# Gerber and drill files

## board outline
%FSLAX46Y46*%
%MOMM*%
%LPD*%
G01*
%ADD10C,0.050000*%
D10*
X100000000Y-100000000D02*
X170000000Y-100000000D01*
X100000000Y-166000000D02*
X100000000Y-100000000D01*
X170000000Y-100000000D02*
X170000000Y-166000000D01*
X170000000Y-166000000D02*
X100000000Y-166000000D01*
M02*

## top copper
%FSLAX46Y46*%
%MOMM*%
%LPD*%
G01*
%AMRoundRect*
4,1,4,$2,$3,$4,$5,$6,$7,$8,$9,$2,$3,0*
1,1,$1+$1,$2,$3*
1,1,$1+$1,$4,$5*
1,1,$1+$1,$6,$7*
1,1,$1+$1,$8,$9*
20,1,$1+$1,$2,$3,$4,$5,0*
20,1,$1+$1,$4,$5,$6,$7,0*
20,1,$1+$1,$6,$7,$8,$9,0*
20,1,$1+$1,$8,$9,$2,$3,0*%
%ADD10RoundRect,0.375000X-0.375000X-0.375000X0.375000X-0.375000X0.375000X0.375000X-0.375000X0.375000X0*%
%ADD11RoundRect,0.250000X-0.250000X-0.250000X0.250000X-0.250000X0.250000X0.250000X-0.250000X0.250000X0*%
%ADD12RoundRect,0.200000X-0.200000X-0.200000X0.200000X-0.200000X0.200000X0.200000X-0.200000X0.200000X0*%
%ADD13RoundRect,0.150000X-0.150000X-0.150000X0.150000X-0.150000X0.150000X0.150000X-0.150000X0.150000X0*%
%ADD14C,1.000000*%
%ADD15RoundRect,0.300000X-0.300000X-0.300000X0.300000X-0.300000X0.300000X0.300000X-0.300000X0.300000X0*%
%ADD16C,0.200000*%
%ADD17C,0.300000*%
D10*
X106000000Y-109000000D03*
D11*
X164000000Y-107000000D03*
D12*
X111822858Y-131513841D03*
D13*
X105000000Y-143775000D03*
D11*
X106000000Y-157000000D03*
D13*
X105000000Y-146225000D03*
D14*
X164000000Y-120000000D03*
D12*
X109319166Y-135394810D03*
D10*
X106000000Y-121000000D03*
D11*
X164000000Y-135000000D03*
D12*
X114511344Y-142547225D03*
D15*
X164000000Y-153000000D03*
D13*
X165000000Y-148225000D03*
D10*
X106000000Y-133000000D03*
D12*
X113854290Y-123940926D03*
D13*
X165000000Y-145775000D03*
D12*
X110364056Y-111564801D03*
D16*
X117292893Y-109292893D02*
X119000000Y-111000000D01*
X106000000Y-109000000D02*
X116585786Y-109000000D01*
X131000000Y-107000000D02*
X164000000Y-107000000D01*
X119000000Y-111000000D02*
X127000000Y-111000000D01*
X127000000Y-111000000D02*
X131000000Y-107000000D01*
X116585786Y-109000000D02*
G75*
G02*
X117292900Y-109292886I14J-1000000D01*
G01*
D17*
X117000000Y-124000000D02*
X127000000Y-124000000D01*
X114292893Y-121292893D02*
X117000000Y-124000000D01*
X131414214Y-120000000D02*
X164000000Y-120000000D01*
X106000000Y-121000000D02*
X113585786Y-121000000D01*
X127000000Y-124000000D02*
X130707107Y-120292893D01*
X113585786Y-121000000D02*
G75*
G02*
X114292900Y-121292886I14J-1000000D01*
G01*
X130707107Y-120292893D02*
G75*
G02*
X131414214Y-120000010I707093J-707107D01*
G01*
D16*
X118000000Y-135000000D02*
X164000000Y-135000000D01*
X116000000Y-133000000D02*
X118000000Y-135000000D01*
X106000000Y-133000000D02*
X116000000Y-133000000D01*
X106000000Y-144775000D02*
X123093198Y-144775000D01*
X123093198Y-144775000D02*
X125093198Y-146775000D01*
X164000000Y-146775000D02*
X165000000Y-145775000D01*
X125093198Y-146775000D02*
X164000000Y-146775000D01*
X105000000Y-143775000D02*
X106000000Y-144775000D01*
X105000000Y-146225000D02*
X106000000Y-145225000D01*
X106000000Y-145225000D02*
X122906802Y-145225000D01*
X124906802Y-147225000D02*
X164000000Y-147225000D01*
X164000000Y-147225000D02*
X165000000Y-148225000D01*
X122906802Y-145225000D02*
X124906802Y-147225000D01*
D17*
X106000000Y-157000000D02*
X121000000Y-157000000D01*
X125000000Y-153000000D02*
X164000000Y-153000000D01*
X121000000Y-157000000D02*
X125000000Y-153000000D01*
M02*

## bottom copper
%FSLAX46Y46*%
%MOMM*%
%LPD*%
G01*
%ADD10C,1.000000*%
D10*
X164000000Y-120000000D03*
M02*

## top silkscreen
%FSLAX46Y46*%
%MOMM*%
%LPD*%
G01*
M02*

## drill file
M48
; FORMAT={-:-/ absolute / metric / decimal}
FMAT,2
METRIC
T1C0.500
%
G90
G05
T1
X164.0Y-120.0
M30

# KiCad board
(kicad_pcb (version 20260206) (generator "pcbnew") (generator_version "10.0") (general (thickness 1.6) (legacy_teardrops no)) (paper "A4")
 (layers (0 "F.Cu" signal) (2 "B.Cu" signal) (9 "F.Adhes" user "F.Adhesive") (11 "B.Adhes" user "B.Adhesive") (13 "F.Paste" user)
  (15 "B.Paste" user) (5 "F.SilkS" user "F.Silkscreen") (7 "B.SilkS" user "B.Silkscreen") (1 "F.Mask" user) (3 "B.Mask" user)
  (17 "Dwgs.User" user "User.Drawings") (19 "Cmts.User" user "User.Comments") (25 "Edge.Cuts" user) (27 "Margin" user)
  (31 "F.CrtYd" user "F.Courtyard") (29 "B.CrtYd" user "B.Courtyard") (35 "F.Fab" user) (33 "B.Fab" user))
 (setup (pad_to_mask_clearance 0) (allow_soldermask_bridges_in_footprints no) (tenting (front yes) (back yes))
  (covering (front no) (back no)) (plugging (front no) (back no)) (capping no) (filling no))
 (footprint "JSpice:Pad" (layer "F.Cu") (at 106 109)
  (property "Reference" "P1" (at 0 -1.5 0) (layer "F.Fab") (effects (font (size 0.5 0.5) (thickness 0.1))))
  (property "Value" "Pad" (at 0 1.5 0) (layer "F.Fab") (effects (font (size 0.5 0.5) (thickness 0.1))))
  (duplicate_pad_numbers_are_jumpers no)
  (pad "1" smd roundrect (at 0 0) (size 1.5 1.5) (layers "F.Cu" "F.Mask") (roundrect_rratio 0.25) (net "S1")))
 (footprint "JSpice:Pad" (layer "F.Cu") (at 164 107)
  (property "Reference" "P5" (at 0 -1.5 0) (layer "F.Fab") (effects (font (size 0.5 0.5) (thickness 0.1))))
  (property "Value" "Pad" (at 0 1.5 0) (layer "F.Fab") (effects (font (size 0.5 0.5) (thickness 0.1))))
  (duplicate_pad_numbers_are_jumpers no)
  (pad "1" smd roundrect (at 0 0) (size 1 1) (layers "F.Cu" "F.Mask") (roundrect_rratio 0.25) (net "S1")))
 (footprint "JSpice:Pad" (layer "F.Cu") (at 111.822858 131.513841)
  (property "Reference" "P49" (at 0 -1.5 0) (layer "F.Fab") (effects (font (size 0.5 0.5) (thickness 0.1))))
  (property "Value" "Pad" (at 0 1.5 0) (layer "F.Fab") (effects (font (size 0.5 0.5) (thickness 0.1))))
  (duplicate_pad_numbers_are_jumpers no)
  (pad "1" smd roundrect (at 0 0) (size 0.8 0.8) (layers "F.Cu" "F.Mask") (roundrect_rratio 0.25) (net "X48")))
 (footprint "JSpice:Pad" (layer "F.Cu") (at 105 143.775)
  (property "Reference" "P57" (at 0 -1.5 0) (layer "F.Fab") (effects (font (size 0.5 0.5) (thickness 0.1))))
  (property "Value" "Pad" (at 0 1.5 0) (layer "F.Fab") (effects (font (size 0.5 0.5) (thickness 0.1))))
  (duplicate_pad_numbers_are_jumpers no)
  (pad "1" smd roundrect (at 0 0) (size 0.6 0.6) (layers "F.Cu" "F.Mask") (roundrect_rratio 0.25) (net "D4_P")))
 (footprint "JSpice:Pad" (layer "F.Cu") (at 106 157)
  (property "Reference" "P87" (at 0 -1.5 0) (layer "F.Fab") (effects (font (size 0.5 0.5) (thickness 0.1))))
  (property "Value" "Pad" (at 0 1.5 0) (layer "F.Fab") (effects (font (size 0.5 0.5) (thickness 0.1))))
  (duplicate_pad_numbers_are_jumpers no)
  (pad "1" smd roundrect (at 0 0) (size 1 1) (layers "F.Cu" "F.Mask") (roundrect_rratio 0.25) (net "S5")))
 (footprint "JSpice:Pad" (layer "F.Cu") (at 105 146.225)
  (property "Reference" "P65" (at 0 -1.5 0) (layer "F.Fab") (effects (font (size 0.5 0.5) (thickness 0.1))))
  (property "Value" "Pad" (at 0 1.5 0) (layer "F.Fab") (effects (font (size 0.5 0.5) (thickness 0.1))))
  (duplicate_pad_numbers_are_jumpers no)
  (pad "1" smd roundrect (at 0 0) (size 0.6 0.6) (layers "F.Cu" "F.Mask") (roundrect_rratio 0.25) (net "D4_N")))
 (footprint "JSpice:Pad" (layer "F.Cu") (at 164 120)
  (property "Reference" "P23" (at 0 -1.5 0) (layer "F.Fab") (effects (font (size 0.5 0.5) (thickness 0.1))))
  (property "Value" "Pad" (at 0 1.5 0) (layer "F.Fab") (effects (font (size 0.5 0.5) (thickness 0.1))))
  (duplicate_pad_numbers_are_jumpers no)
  (pad "1" thru_hole circle (at 0 0) (size 1 1) (drill 0.5) (layers "*.Cu" "*.Mask") (remove_unused_layers no) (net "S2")))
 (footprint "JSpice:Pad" (layer "F.Cu") (at 109.319166 135.39481)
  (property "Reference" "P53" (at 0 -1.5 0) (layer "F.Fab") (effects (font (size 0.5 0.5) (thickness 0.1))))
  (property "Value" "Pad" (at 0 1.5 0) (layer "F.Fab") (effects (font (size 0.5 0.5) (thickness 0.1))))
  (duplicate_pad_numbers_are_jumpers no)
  (pad "1" smd roundrect (at 0 0) (size 0.8 0.8) (layers "F.Cu" "F.Mask") (roundrect_rratio 0.25) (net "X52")))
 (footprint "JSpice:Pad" (layer "F.Cu") (at 106 121)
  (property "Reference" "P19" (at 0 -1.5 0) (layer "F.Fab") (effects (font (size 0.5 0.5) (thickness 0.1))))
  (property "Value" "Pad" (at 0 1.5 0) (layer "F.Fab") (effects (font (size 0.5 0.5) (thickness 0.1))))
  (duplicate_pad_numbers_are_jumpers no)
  (pad "1" smd roundrect (at 0 0) (size 1.5 1.5) (layers "F.Cu" "F.Mask") (roundrect_rratio 0.25) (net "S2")))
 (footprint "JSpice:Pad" (layer "F.Cu") (at 164 135)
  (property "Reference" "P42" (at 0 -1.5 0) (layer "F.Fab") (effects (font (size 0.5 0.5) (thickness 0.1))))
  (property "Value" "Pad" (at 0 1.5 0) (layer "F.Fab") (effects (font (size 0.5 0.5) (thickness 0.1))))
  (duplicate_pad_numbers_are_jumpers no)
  (pad "1" smd roundrect (at 0 0) (size 1 1) (layers "F.Cu" "F.Mask") (roundrect_rratio 0.25) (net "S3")))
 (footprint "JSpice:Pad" (layer "F.Cu") (at 114.511344 142.547225)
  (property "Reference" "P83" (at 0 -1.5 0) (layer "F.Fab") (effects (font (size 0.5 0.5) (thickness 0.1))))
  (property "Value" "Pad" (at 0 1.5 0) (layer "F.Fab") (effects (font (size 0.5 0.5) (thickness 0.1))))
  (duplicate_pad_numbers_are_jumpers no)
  (pad "1" smd roundrect (at 0 0) (size 0.8 0.8) (layers "F.Cu" "F.Mask") (roundrect_rratio 0.25) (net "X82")))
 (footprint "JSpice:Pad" (layer "F.Cu") (at 164 153)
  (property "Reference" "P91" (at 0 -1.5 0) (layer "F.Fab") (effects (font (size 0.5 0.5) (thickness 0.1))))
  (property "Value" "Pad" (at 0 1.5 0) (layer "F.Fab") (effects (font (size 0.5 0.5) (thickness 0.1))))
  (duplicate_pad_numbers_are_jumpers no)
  (pad "1" smd roundrect (at 0 0) (size 1.2 1.2) (layers "F.Cu" "F.Mask") (roundrect_rratio 0.25) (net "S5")))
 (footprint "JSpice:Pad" (layer "F.Cu") (at 165 148.225)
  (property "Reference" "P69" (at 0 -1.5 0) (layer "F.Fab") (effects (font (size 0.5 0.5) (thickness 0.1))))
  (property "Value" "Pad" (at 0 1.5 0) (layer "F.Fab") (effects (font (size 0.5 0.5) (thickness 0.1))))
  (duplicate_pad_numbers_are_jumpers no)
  (pad "1" smd roundrect (at 0 0) (size 0.6 0.6) (layers "F.Cu" "F.Mask") (roundrect_rratio 0.25) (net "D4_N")))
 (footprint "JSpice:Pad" (layer "F.Cu") (at 106 133)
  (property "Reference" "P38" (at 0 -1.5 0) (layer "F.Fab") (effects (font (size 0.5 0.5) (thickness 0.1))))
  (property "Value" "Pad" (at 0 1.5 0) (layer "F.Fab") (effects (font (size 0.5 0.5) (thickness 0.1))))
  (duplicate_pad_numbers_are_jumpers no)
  (pad "1" smd roundrect (at 0 0) (size 1.5 1.5) (layers "F.Cu" "F.Mask") (roundrect_rratio 0.25) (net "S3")))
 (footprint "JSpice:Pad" (layer "F.Cu") (at 113.85429 123.940926)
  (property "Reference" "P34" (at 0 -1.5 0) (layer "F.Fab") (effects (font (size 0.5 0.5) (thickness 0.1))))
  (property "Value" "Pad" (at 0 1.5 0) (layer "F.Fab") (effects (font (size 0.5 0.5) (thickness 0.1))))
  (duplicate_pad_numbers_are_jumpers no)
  (pad "1" smd roundrect (at 0 0) (size 0.8 0.8) (layers "F.Cu" "F.Mask") (roundrect_rratio 0.25) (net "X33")))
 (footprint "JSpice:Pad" (layer "F.Cu") (at 165 145.775)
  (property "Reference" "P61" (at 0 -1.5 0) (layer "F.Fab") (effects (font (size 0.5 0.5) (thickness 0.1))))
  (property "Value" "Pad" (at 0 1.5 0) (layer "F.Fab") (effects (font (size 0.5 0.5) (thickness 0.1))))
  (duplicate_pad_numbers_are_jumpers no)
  (pad "1" smd roundrect (at 0 0) (size 0.6 0.6) (layers "F.Cu" "F.Mask") (roundrect_rratio 0.25) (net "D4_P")))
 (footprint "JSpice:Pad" (layer "F.Cu") (at 110.364056 111.564801)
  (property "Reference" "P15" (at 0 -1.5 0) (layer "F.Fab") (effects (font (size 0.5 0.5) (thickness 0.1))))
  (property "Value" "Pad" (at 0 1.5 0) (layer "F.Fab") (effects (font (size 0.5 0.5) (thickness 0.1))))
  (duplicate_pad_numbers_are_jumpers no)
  (pad "1" smd roundrect (at 0 0) (size 0.8 0.8) (layers "F.Cu" "F.Mask") (roundrect_rratio 0.25) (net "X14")))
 (gr_line (start 100 100) (end 170 100) (stroke (width 0.05) (type default)) (layer "Edge.Cuts"))
 (gr_line (start 100 166) (end 100 100) (stroke (width 0.05) (type default)) (layer "Edge.Cuts"))
 (gr_line (start 170 100) (end 170 166) (stroke (width 0.05) (type default)) (layer "Edge.Cuts"))
 (gr_line (start 170 166) (end 100 166) (stroke (width 0.05) (type default)) (layer "Edge.Cuts"))
 (segment (start 117.292893 109.292893) (end 119 111) (width 0.2) (layer "F.Cu") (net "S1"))
 (segment (start 106 109) (end 116.585786 109) (width 0.2) (layer "F.Cu") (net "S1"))
 (segment (start 131 107) (end 164 107) (width 0.2) (layer "F.Cu") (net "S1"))
 (segment (start 119 111) (end 127 111) (width 0.2) (layer "F.Cu") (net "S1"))
 (segment (start 127 111) (end 131 107) (width 0.2) (layer "F.Cu") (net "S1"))
 (arc (start 116.585786 109) (mid 116.96847 109.07612) (end 117.292893 109.292893) (width 0.2) (layer "F.Cu") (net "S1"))
 (segment (start 117 124) (end 127 124) (width 0.3) (layer "F.Cu") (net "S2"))
 (segment (start 114.292893 121.292893) (end 117 124) (width 0.3) (layer "F.Cu") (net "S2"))
 (segment (start 131.414214 120) (end 164 120) (width 0.3) (layer "F.Cu") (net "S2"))
 (segment (start 106 121) (end 113.585786 121) (width 0.3) (layer "F.Cu") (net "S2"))
 (segment (start 127 124) (end 130.707107 120.292893) (width 0.3) (layer "F.Cu") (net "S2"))
 (arc (start 113.585786 121) (mid 113.96847 121.07612) (end 114.292893 121.292893) (width 0.3) (layer "F.Cu") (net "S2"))
 (arc (start 130.707107 120.292893) (mid 131.03153 120.07612) (end 131.414214 120) (width 0.3) (layer "F.Cu") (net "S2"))
 (segment (start 118 135) (end 164 135) (width 0.2) (layer "F.Cu") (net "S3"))
 (segment (start 116 133) (end 118 135) (width 0.2) (layer "F.Cu") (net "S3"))
 (segment (start 106 133) (end 116 133) (width 0.2) (layer "F.Cu") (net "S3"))
 (segment (start 106 144.775) (end 123.093198 144.775) (width 0.2) (layer "F.Cu") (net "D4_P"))
 (segment (start 123.093198 144.775) (end 125.093198 146.775) (width 0.2) (layer "F.Cu") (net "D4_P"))
 (segment (start 164 146.775) (end 165 145.775) (width 0.2) (layer "F.Cu") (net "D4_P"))
 (segment (start 125.093198 146.775) (end 164 146.775) (width 0.2) (layer "F.Cu") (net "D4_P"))
 (segment (start 105 143.775) (end 106 144.775) (width 0.2) (layer "F.Cu") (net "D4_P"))
 (segment (start 105 146.225) (end 106 145.225) (width 0.2) (layer "F.Cu") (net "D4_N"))
 (segment (start 106 145.225) (end 122.906802 145.225) (width 0.2) (layer "F.Cu") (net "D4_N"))
 (segment (start 124.906802 147.225) (end 164 147.225) (width 0.2) (layer "F.Cu") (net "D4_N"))
 (segment (start 164 147.225) (end 165 148.225) (width 0.2) (layer "F.Cu") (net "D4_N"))
 (segment (start 122.906802 145.225) (end 124.906802 147.225) (width 0.2) (layer "F.Cu") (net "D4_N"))
 (segment (start 106 157) (end 121 157) (width 0.3) (layer "F.Cu") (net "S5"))
 (segment (start 125 153) (end 164 153) (width 0.3) (layer "F.Cu") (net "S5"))
 (segment (start 121 157) (end 125 153) (width 0.3) (layer "F.Cu") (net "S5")))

